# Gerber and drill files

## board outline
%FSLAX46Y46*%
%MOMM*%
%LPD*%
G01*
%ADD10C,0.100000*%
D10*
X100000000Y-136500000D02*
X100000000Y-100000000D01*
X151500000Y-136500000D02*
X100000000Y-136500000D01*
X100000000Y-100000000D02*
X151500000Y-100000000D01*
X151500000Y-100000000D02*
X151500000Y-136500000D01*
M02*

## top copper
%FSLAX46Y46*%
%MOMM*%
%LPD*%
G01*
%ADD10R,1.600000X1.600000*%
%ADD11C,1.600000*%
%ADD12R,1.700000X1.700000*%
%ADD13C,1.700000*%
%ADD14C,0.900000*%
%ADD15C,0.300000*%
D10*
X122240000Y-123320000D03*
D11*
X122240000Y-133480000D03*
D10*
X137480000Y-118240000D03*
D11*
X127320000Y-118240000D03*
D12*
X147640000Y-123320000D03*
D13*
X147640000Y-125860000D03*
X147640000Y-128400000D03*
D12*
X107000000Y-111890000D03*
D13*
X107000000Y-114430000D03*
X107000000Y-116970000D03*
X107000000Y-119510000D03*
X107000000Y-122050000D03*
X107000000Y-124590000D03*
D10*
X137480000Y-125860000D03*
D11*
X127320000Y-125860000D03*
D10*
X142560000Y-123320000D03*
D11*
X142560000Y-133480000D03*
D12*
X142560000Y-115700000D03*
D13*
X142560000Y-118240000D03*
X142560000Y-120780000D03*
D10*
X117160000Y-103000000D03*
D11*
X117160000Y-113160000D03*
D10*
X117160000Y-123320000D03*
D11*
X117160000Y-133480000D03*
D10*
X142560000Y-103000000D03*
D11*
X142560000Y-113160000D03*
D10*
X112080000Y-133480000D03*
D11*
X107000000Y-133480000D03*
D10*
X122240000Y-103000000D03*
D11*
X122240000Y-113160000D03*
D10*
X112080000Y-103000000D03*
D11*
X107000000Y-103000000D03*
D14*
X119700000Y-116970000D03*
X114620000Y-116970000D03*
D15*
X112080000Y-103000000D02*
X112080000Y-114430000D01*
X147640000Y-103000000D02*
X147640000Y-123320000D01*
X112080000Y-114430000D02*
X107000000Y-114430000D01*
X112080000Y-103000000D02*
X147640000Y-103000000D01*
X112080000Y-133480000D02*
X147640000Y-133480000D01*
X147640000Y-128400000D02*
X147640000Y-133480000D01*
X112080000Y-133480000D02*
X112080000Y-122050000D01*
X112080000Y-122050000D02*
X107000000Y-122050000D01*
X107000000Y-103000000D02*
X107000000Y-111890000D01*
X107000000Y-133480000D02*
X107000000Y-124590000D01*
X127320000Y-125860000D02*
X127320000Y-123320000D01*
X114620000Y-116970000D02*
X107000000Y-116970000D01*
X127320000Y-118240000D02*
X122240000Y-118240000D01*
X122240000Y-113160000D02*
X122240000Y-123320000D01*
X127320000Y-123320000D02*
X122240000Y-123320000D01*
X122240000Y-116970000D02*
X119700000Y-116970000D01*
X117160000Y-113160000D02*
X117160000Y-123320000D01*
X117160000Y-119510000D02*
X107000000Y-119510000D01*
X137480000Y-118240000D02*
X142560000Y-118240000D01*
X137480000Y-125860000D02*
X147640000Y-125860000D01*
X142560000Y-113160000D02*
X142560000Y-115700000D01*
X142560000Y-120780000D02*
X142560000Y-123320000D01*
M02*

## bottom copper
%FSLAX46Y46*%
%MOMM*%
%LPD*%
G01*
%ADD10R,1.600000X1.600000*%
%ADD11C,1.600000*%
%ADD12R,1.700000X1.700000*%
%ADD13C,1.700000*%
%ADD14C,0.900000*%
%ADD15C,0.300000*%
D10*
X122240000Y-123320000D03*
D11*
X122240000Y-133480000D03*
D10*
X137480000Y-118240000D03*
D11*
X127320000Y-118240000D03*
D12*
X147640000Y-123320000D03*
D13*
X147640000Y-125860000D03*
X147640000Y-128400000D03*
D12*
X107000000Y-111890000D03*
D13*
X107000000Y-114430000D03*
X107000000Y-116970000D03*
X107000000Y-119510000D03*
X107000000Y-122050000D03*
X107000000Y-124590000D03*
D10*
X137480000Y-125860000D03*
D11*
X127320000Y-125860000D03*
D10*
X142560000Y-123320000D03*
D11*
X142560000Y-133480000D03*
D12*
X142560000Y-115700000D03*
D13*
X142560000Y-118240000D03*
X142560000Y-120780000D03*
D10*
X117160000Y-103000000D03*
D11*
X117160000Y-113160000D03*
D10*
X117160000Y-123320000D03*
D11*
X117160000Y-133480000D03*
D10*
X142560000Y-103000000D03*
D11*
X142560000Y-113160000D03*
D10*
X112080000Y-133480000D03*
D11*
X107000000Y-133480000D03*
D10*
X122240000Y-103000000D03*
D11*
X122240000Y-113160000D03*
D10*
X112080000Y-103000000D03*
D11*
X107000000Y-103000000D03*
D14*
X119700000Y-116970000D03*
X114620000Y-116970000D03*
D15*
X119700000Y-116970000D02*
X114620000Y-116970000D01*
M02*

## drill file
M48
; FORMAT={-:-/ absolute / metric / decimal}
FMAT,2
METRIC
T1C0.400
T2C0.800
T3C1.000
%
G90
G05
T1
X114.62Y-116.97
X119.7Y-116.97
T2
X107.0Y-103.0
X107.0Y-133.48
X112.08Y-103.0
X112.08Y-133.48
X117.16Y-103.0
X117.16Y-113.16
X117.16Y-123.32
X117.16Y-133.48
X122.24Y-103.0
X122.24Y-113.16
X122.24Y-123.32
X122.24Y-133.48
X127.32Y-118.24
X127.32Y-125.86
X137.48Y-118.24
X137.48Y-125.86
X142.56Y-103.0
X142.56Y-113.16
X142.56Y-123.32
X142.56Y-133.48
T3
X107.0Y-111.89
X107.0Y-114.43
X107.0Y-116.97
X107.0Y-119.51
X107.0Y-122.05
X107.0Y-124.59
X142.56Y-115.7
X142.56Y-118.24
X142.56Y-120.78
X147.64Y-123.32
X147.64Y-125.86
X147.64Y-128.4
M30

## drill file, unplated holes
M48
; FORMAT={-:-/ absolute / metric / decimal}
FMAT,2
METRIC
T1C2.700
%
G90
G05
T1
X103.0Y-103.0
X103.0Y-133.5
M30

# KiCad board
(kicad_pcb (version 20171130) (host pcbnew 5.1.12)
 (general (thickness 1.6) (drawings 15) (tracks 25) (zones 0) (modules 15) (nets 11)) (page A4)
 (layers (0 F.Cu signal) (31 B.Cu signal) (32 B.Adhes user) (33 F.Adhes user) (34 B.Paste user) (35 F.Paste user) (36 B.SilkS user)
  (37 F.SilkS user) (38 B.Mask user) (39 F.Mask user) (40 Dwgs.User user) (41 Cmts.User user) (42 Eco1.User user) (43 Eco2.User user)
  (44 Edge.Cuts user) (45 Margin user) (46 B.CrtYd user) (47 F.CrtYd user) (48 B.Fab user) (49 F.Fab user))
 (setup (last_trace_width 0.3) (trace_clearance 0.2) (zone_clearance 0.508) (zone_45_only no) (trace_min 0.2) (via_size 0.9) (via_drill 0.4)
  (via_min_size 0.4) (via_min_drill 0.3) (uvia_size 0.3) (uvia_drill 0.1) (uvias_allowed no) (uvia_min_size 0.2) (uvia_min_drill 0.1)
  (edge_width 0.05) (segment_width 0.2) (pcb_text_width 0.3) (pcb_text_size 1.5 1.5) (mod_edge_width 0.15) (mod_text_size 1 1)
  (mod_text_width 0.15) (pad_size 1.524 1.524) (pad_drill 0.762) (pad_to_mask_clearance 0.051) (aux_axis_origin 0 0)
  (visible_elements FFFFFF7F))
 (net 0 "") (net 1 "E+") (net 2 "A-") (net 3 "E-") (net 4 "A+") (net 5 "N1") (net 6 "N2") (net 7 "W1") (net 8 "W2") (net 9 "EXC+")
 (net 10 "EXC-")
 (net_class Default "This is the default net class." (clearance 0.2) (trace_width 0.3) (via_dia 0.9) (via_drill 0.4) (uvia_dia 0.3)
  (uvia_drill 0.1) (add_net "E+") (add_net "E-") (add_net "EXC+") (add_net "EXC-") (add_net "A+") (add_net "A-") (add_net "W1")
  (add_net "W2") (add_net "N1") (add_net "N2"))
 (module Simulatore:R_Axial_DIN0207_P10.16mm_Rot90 (layer F.Cu) (at 117.16 103)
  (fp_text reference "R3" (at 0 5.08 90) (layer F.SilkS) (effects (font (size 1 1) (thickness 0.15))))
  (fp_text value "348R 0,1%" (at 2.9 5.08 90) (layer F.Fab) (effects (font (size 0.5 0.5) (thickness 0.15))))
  (pad 1 thru_hole rect (at 0 0) (size 1.6 1.6) (drill 0.8) (layers *.Cu *.Mask) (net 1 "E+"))
  (pad 2 thru_hole circle (at 0 10.16) (size 1.6 1.6) (drill 0.8) (layers *.Cu *.Mask) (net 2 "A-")))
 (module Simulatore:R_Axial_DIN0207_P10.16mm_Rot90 (layer F.Cu) (at 117.16 123.32)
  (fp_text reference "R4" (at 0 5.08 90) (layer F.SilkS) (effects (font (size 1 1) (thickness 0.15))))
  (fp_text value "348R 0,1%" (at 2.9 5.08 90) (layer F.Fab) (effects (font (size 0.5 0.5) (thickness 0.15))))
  (pad 1 thru_hole rect (at 0 0) (size 1.6 1.6) (drill 0.8) (layers *.Cu *.Mask) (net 2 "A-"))
  (pad 2 thru_hole circle (at 0 10.16) (size 1.6 1.6) (drill 0.8) (layers *.Cu *.Mask) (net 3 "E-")))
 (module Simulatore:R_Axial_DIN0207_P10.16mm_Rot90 (layer F.Cu) (at 122.24 103)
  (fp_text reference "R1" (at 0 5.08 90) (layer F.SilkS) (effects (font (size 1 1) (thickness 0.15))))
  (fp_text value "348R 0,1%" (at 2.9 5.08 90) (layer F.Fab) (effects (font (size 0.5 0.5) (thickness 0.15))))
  (pad 1 thru_hole rect (at 0 0) (size 1.6 1.6) (drill 0.8) (layers *.Cu *.Mask) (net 1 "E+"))
  (pad 2 thru_hole circle (at 0 10.16) (size 1.6 1.6) (drill 0.8) (layers *.Cu *.Mask) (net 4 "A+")))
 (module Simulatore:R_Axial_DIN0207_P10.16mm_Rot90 (layer F.Cu) (at 122.24 123.32)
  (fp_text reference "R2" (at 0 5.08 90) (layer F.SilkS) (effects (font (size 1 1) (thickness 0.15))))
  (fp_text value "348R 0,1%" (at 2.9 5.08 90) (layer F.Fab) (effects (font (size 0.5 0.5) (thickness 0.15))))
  (pad 1 thru_hole rect (at 0 0) (size 1.6 1.6) (drill 0.8) (layers *.Cu *.Mask) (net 4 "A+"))
  (pad 2 thru_hole circle (at 0 10.16) (size 1.6 1.6) (drill 0.8) (layers *.Cu *.Mask) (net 3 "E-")))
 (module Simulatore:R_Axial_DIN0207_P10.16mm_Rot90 (layer F.Cu) (at 142.56 103)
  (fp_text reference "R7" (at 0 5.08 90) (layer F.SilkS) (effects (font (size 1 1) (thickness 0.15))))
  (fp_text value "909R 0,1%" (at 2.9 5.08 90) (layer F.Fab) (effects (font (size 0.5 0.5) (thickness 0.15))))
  (pad 1 thru_hole rect (at 0 0) (size 1.6 1.6) (drill 0.8) (layers *.Cu *.Mask) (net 1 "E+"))
  (pad 2 thru_hole circle (at 0 10.16) (size 1.6 1.6) (drill 0.8) (layers *.Cu *.Mask) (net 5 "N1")))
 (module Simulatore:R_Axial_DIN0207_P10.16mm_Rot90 (layer F.Cu) (at 142.56 123.32)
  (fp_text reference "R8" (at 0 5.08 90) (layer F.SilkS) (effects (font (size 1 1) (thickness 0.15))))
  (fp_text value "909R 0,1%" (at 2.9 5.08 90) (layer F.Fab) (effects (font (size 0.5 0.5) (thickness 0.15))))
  (pad 1 thru_hole rect (at 0 0) (size 1.6 1.6) (drill 0.8) (layers *.Cu *.Mask) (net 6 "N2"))
  (pad 2 thru_hole circle (at 0 10.16) (size 1.6 1.6) (drill 0.8) (layers *.Cu *.Mask) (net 3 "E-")))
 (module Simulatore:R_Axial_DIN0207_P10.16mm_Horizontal (layer F.Cu) (at 132.4 118.24)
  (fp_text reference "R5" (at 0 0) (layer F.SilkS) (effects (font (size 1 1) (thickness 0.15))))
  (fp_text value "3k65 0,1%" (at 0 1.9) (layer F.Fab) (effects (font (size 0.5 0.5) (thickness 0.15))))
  (pad 1 thru_hole rect (at 5.08 0) (size 1.6 1.6) (drill 0.8) (layers *.Cu *.Mask) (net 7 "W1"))
  (pad 2 thru_hole circle (at -5.08 0) (size 1.6 1.6) (drill 0.8) (layers *.Cu *.Mask) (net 4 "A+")))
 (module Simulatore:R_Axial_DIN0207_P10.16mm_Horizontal (layer F.Cu) (at 132.4 125.86)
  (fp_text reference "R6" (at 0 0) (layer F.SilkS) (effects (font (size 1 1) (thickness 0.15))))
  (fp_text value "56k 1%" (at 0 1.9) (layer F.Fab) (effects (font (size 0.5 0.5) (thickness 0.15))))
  (pad 1 thru_hole rect (at 5.08 0) (size 1.6 1.6) (drill 0.8) (layers *.Cu *.Mask) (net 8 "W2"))
  (pad 2 thru_hole circle (at -5.08 0) (size 1.6 1.6) (drill 0.8) (layers *.Cu *.Mask) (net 4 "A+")))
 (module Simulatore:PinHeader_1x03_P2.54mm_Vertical (layer F.Cu) (at 142.56 115.7)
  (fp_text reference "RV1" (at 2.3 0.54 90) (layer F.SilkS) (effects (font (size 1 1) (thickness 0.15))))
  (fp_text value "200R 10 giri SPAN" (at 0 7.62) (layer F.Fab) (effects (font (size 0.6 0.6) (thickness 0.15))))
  (pad 1 thru_hole rect (at 0 0) (size 1.7 1.7) (drill 1) (layers *.Cu *.Mask) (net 5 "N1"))
  (pad 2 thru_hole circle (at 0 2.54) (size 1.7 1.7) (drill 1) (layers *.Cu *.Mask) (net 7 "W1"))
  (pad 3 thru_hole circle (at 0 5.08) (size 1.7 1.7) (drill 1) (layers *.Cu *.Mask) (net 6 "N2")))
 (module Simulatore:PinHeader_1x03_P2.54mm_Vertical (layer F.Cu) (at 147.64 123.32)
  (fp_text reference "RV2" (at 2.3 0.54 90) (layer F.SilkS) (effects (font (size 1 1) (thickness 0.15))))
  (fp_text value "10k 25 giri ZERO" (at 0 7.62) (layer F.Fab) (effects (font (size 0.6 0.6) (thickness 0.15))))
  (pad 1 thru_hole rect (at 0 0) (size 1.7 1.7) (drill 1) (layers *.Cu *.Mask) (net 1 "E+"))
  (pad 2 thru_hole circle (at 0 2.54) (size 1.7 1.7) (drill 1) (layers *.Cu *.Mask) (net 8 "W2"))
  (pad 3 thru_hole circle (at 0 5.08) (size 1.7 1.7) (drill 1) (layers *.Cu *.Mask) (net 3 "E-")))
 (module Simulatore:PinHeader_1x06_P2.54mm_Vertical (layer F.Cu) (at 107 111.89)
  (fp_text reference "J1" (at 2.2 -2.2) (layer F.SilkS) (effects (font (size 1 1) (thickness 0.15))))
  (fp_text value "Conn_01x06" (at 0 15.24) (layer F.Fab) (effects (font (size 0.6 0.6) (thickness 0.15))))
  (pad 1 thru_hole rect (at 0 0) (size 1.7 1.7) (drill 1) (layers *.Cu *.Mask) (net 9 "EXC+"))
  (pad 2 thru_hole circle (at 0 2.54) (size 1.7 1.7) (drill 1) (layers *.Cu *.Mask) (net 1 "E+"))
  (pad 3 thru_hole circle (at 0 5.08) (size 1.7 1.7) (drill 1) (layers *.Cu *.Mask) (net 4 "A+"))
  (pad 4 thru_hole circle (at 0 7.62) (size 1.7 1.7) (drill 1) (layers *.Cu *.Mask) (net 2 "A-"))
  (pad 5 thru_hole circle (at 0 10.16) (size 1.7 1.7) (drill 1) (layers *.Cu *.Mask) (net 3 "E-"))
  (pad 6 thru_hole circle (at 0 12.7) (size 1.7 1.7) (drill 1) (layers *.Cu *.Mask) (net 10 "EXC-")))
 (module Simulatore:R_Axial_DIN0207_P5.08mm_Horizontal (layer F.Cu) (at 112.08 103)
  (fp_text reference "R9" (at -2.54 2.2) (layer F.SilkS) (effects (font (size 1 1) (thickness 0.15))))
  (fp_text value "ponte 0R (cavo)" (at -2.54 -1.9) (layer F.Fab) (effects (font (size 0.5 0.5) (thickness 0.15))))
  (pad 1 thru_hole rect (at 0 0) (size 1.6 1.6) (drill 0.8) (layers *.Cu *.Mask) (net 1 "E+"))
  (pad 2 thru_hole circle (at -5.08 0) (size 1.6 1.6) (drill 0.8) (layers *.Cu *.Mask) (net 9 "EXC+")))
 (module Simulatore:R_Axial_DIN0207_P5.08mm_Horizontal (layer F.Cu) (at 112.08 133.48)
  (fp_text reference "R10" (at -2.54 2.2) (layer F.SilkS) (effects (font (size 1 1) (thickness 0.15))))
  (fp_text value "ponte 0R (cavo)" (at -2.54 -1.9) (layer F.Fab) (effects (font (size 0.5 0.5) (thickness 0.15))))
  (pad 1 thru_hole rect (at 0 0) (size 1.6 1.6) (drill 0.8) (layers *.Cu *.Mask) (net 3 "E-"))
  (pad 2 thru_hole circle (at -5.08 0) (size 1.6 1.6) (drill 0.8) (layers *.Cu *.Mask) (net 10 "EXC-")))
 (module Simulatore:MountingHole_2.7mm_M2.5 (layer F.Cu) (at 103 103)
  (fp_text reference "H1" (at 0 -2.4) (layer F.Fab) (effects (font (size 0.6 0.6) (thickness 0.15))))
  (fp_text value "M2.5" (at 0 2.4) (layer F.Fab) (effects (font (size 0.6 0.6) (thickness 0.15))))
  (pad "" np_thru_hole circle (at 0 0) (size 2.7 2.7) (drill 2.7) (layers *.Cu *.Mask)))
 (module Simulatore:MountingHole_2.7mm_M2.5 (layer F.Cu) (at 103 133.5)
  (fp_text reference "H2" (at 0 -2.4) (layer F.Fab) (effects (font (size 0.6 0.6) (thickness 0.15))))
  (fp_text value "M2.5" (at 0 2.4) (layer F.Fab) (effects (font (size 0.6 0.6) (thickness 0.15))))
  (pad "" np_thru_hole circle (at 0 0) (size 2.7 2.7) (drill 2.7) (layers *.Cu *.Mask)))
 (gr_line (start 100 100) (end 151.5 100) (layer Edge.Cuts) (width 0.05))
 (gr_line (start 151.5 100) (end 151.5 136.5) (layer Edge.Cuts) (width 0.05))
 (gr_line (start 151.5 136.5) (end 100 136.5) (layer Edge.Cuts) (width 0.05))
 (gr_line (start 100 136.5) (end 100 100) (layer Edge.Cuts) (width 0.05))
 (segment (start 112.08 103) (end 147.64 103) (width 0.3) (layer F.Cu) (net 1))
 (segment (start 112.08 133.48) (end 147.64 133.48) (width 0.3) (layer F.Cu) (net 3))
 (segment (start 107 103) (end 107 111.89) (width 0.3) (layer F.Cu) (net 9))
 (segment (start 107 133.48) (end 107 124.59) (width 0.3) (layer F.Cu) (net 10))
 (segment (start 112.08 103) (end 112.08 114.43) (width 0.3) (layer F.Cu) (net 1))
 (segment (start 112.08 114.43) (end 107 114.43) (width 0.3) (layer F.Cu) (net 1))
 (segment (start 112.08 133.48) (end 112.08 122.05) (width 0.3) (layer F.Cu) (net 3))
 (segment (start 112.08 122.05) (end 107 122.05) (width 0.3) (layer F.Cu) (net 3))
 (segment (start 117.16 113.16) (end 117.16 123.32) (width 0.3) (layer F.Cu) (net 2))
 (segment (start 117.16 119.51) (end 107 119.51) (width 0.3) (layer F.Cu) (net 2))
 (segment (start 122.24 113.16) (end 122.24 123.32) (width 0.3) (layer F.Cu) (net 4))
 (segment (start 122.24 116.97) (end 119.7 116.97) (width 0.3) (layer F.Cu) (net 4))
 (segment (start 119.7 116.97) (end 114.62 116.97) (width 0.3) (layer B.Cu) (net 4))
 (segment (start 114.62 116.97) (end 107 116.97) (width 0.3) (layer F.Cu) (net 4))
 (segment (start 127.32 118.24) (end 122.24 118.24) (width 0.3) (layer F.Cu) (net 4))
 (segment (start 127.32 125.86) (end 127.32 123.32) (width 0.3) (layer F.Cu) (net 4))
 (segment (start 127.32 123.32) (end 122.24 123.32) (width 0.3) (layer F.Cu) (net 4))
 (segment (start 137.48 118.24) (end 142.56 118.24) (width 0.3) (layer F.Cu) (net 7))
 (segment (start 137.48 125.86) (end 147.64 125.86) (width 0.3) (layer F.Cu) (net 8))
 (segment (start 142.56 113.16) (end 142.56 115.7) (width 0.3) (layer F.Cu) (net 5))
 (segment (start 142.56 120.78) (end 142.56 123.32) (width 0.3) (layer F.Cu) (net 6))
 (segment (start 147.64 103) (end 147.64 123.32) (width 0.3) (layer F.Cu) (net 1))
 (segment (start 147.64 128.4) (end 147.64 133.48) (width 0.3) (layer F.Cu) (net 3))
 (via (at 119.7 116.97) (size 0.9) (drill 0.4) (layers F.Cu B.Cu) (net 4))
 (via (at 114.62 116.97) (size 0.9) (drill 0.4) (layers F.Cu B.Cu) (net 4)))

